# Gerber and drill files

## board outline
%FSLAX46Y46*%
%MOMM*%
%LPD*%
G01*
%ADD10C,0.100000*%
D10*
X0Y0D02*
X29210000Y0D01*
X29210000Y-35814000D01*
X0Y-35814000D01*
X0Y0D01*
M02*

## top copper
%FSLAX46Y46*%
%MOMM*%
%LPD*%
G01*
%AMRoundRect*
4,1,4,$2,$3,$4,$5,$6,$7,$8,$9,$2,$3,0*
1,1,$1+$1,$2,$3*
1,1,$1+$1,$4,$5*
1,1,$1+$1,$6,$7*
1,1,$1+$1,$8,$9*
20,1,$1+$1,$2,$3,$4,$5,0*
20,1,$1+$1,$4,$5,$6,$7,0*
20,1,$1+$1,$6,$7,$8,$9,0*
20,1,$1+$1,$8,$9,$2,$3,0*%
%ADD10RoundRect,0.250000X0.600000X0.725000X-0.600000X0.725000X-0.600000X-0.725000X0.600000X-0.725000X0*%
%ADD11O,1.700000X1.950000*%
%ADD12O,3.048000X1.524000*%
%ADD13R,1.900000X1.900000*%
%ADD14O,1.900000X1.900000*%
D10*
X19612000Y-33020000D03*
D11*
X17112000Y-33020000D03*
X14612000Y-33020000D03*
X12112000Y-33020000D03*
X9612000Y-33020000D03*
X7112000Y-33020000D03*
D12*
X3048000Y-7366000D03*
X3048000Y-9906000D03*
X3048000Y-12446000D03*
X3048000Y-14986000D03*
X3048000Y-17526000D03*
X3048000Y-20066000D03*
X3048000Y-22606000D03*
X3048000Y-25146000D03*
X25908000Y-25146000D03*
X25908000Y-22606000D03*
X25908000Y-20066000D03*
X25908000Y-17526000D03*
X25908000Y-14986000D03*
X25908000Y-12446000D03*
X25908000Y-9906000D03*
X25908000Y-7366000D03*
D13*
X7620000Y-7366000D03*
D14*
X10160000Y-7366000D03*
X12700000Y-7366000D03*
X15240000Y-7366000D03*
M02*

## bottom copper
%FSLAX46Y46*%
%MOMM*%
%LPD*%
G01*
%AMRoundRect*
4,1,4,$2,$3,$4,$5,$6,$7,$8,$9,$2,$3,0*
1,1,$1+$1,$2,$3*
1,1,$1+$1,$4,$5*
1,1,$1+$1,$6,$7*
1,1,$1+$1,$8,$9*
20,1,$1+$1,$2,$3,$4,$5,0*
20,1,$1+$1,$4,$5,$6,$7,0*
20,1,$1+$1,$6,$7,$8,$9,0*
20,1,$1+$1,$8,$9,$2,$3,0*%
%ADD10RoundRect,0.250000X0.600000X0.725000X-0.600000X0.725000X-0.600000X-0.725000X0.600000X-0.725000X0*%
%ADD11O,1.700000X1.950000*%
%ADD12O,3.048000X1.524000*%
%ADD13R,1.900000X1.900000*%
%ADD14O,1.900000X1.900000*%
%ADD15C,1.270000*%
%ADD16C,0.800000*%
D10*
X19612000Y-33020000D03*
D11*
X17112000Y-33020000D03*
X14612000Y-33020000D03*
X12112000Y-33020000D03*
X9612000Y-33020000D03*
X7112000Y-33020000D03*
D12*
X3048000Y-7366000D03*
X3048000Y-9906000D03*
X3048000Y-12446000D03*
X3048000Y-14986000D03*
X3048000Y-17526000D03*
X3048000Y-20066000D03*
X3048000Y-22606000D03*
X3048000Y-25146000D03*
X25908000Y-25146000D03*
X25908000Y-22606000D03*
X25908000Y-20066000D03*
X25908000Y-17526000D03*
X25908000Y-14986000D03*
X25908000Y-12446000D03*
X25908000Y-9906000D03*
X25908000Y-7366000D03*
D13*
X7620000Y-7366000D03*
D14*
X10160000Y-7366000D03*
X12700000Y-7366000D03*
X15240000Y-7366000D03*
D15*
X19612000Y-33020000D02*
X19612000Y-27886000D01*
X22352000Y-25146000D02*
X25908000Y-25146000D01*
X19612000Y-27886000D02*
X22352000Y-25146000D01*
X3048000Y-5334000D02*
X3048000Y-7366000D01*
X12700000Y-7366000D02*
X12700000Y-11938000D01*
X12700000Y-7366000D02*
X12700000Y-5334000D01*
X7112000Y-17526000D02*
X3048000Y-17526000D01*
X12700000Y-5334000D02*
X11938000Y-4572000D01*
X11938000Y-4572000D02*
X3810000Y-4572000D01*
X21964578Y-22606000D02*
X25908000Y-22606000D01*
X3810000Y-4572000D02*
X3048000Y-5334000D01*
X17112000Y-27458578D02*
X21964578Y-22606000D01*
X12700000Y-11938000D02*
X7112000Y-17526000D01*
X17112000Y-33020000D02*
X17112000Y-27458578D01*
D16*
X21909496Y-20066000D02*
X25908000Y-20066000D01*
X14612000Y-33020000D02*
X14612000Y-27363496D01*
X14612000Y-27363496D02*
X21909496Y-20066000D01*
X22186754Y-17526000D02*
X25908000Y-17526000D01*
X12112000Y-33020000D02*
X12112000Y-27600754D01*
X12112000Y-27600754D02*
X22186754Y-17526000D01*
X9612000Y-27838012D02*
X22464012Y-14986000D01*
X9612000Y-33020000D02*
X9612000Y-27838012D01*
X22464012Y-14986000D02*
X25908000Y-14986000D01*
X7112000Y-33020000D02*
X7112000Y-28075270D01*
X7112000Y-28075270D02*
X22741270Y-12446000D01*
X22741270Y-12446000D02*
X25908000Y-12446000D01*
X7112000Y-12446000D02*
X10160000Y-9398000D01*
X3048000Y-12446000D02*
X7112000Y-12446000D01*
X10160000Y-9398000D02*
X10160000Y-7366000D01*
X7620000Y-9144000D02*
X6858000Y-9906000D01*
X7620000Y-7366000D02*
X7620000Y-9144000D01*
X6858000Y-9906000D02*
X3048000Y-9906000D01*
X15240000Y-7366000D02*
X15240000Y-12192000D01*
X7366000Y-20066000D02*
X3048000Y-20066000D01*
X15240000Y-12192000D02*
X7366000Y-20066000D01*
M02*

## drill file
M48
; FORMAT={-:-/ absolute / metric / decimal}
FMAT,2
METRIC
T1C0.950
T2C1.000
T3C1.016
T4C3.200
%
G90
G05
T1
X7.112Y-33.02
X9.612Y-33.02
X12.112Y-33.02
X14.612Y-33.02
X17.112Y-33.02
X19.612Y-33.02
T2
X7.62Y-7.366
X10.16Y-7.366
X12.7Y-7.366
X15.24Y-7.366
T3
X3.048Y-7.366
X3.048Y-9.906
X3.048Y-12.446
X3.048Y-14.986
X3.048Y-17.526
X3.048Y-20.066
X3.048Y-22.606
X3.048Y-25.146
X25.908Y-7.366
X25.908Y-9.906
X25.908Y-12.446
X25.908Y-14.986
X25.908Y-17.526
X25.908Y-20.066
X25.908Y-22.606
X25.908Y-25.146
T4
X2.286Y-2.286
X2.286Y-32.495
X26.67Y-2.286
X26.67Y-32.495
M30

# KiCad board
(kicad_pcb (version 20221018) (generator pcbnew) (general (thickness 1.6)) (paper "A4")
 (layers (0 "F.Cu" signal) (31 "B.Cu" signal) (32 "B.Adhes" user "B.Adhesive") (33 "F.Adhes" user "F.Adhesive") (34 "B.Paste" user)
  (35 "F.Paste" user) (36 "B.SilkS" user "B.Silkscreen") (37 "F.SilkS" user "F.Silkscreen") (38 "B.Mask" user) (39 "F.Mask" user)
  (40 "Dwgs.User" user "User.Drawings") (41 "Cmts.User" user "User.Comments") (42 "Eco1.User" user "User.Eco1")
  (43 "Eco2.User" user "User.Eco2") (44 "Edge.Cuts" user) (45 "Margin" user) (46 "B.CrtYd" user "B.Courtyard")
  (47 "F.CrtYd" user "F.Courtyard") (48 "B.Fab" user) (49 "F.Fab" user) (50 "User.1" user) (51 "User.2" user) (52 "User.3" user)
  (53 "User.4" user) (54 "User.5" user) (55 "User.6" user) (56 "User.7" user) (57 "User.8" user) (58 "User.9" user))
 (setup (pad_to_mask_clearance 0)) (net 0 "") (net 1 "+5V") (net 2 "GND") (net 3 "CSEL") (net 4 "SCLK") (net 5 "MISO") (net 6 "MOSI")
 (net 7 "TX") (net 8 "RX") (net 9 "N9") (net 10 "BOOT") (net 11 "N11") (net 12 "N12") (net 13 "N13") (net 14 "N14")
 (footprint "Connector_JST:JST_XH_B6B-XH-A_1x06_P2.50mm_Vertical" (layer "F.Cu") (at 19.612 33.02 180)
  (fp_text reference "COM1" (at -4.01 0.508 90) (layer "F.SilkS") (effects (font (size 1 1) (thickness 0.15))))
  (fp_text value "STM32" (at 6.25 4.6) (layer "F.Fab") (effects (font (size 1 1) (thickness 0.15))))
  (pad "1" thru_hole roundrect (at 0 0 180) (size 1.7 1.95) (drill 0.95) (layers "*.Cu" "*.Mask") (roundrect_rratio 0.1470588235)
   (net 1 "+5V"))
  (pad "2" thru_hole oval (at 2.5 0 180) (size 1.7 1.95) (drill 0.95) (layers "*.Cu" "*.Mask") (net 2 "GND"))
  (pad "3" thru_hole oval (at 5 0 180) (size 1.7 1.95) (drill 0.95) (layers "*.Cu" "*.Mask") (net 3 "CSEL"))
  (pad "4" thru_hole oval (at 7.5 0 180) (size 1.7 1.95) (drill 0.95) (layers "*.Cu" "*.Mask") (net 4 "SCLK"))
  (pad "5" thru_hole oval (at 10 0 180) (size 1.7 1.95) (drill 0.95) (layers "*.Cu" "*.Mask") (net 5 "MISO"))
  (pad "6" thru_hole oval (at 12.5 0 180) (size 1.7 1.95) (drill 0.95) (layers "*.Cu" "*.Mask") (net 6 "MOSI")))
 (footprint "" (layer "F.Cu") (at 26.67 2.286)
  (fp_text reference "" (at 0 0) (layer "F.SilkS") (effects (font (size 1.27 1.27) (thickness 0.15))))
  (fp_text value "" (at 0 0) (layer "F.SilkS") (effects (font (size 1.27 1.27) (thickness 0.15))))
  (pad "" np_thru_hole circle (at 0 0) (size 3.2 3.2) (drill 3.2) (layers "F&B.Cu" "*.Mask")))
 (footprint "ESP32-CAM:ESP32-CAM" (layer "F.Cu") (at 14.478 14.986)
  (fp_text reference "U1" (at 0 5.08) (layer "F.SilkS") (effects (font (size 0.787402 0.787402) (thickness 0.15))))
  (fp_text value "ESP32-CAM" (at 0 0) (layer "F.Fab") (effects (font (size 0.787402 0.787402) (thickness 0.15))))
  (pad "P$1" thru_hole oval (at -11.43 -7.62) (size 3.048 1.524) (drill 1.016) (layers "*.Cu" "*.Mask") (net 2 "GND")
   (solder_mask_margin 0.102))
  (pad "P$2" thru_hole oval (at -11.43 -5.08) (size 3.048 1.524) (drill 1.016) (layers "*.Cu" "*.Mask") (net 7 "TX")
   (solder_mask_margin 0.102))
  (pad "P$3" thru_hole oval (at -11.43 -2.54) (size 3.048 1.524) (drill 1.016) (layers "*.Cu" "*.Mask") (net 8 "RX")
   (solder_mask_margin 0.102))
  (pad "P$4" thru_hole oval (at -11.43 0) (size 3.048 1.524) (drill 1.016) (layers "*.Cu" "*.Mask") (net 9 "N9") (solder_mask_margin 0.102))
  (pad "P$5" thru_hole oval (at -11.43 2.54) (size 3.048 1.524) (drill 1.016) (layers "*.Cu" "*.Mask") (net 2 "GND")
   (solder_mask_margin 0.102))
  (pad "P$6" thru_hole oval (at -11.43 5.08) (size 3.048 1.524) (drill 1.016) (layers "*.Cu" "*.Mask") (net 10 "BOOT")
   (solder_mask_margin 0.102))
  (pad "P$7" thru_hole oval (at -11.43 7.62) (size 3.048 1.524) (drill 1.016) (layers "*.Cu" "*.Mask") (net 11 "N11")
   (solder_mask_margin 0.102))
  (pad "P$8" thru_hole oval (at -11.43 10.16) (size 3.048 1.524) (drill 1.016) (layers "*.Cu" "*.Mask") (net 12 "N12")
   (solder_mask_margin 0.102))
  (pad "P$9" thru_hole oval (at 11.43 10.16) (size 3.048 1.524) (drill 1.016) (layers "*.Cu" "*.Mask") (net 1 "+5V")
   (solder_mask_margin 0.102))
  (pad "P$10" thru_hole oval (at 11.43 7.62) (size 3.048 1.524) (drill 1.016) (layers "*.Cu" "*.Mask") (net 2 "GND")
   (solder_mask_margin 0.102))
  (pad "P$11" thru_hole oval (at 11.43 5.08) (size 3.048 1.524) (drill 1.016) (layers "*.Cu" "*.Mask") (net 3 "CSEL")
   (solder_mask_margin 0.102))
  (pad "P$12" thru_hole oval (at 11.43 2.54) (size 3.048 1.524) (drill 1.016) (layers "*.Cu" "*.Mask") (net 4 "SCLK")
   (solder_mask_margin 0.102))
  (pad "P$13" thru_hole oval (at 11.43 0) (size 3.048 1.524) (drill 1.016) (layers "*.Cu" "*.Mask") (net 5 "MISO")
   (solder_mask_margin 0.102))
  (pad "P$14" thru_hole oval (at 11.43 -2.54) (size 3.048 1.524) (drill 1.016) (layers "*.Cu" "*.Mask") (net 6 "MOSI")
   (solder_mask_margin 0.102))
  (pad "P$15" thru_hole oval (at 11.43 -5.08) (size 3.048 1.524) (drill 1.016) (layers "*.Cu" "*.Mask") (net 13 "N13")
   (solder_mask_margin 0.102))
  (pad "P$16" thru_hole oval (at 11.43 -7.62) (size 3.048 1.524) (drill 1.016) (layers "*.Cu" "*.Mask") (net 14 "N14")
   (solder_mask_margin 0.102)))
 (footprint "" (layer "F.Cu") (at 2.286 2.286)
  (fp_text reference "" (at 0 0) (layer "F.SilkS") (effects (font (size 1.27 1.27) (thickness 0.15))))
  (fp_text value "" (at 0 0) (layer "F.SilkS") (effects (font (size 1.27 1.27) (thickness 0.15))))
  (pad "" np_thru_hole circle (at 0 0) (size 3.2 3.2) (drill 3.2) (layers "F&B.Cu" "*.Mask")))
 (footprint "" (layer "F.Cu") (at 26.67 32.495)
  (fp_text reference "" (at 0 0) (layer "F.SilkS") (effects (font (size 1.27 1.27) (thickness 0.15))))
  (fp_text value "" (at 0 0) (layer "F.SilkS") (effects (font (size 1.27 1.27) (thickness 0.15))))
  (pad "" np_thru_hole circle (at 0 0) (size 3.2 3.2) (drill 3.2) (layers "F&B.Cu" "*.Mask")))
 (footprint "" (layer "F.Cu") (at 2.286 32.495)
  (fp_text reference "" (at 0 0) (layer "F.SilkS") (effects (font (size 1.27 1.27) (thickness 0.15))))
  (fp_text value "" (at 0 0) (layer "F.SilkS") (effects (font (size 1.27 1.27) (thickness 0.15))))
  (pad "" np_thru_hole circle (at 0 0) (size 3.2 3.2) (drill 3.2) (layers "F&B.Cu" "*.Mask")))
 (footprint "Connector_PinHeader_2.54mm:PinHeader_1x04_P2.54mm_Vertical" (layer "F.Cu") (at 7.62 7.366 90)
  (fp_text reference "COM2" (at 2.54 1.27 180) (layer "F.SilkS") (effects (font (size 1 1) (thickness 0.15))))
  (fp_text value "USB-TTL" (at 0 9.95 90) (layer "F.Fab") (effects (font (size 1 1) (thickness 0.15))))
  (pad "1" thru_hole rect (at 0 0 90) (size 1.9 1.9) (drill 1) (layers "*.Cu" "*.Mask") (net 7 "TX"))
  (pad "2" thru_hole oval (at 0 2.54 90) (size 1.9 1.9) (drill 1) (layers "*.Cu" "*.Mask") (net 8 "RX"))
  (pad "3" thru_hole oval (at 0 5.08 90) (size 1.9 1.9) (drill 1) (layers "*.Cu" "*.Mask") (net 2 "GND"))
  (pad "4" thru_hole oval (at 0 7.62 90) (size 1.9 1.9) (drill 1) (layers "*.Cu" "*.Mask") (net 10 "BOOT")))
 (gr_rect (start 0 0) (end 29.21 35.814) (stroke (width 0.1) (type default)) (fill none) (layer "Edge.Cuts"))
 (segment (start 19.612 33.02) (end 19.612 27.886) (width 1.27) (layer "B.Cu") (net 1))
 (segment (start 22.352 25.146) (end 25.908 25.146) (width 1.27) (layer "B.Cu") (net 1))
 (segment (start 19.612 27.886) (end 22.352 25.146) (width 1.27) (layer "B.Cu") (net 1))
 (segment (start 3.048 5.334) (end 3.048 7.366) (width 1.27) (layer "B.Cu") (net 2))
 (segment (start 12.7 7.366) (end 12.7 11.938) (width 1.27) (layer "B.Cu") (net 2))
 (segment (start 12.7 7.366) (end 12.7 5.334) (width 1.27) (layer "B.Cu") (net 2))
 (segment (start 7.112 17.526) (end 3.048 17.526) (width 1.27) (layer "B.Cu") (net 2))
 (segment (start 12.7 5.334) (end 11.938 4.572) (width 1.27) (layer "B.Cu") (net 2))
 (segment (start 11.938 4.572) (end 3.81 4.572) (width 1.27) (layer "B.Cu") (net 2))
 (segment (start 21.964578 22.606) (end 25.908 22.606) (width 1.27) (layer "B.Cu") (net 2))
 (segment (start 3.81 4.572) (end 3.048 5.334) (width 1.27) (layer "B.Cu") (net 2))
 (segment (start 17.112 27.458578) (end 21.964578 22.606) (width 1.27) (layer "B.Cu") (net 2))
 (segment (start 12.7 11.938) (end 7.112 17.526) (width 1.27) (layer "B.Cu") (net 2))
 (segment (start 17.112 33.02) (end 17.112 27.458578) (width 1.27) (layer "B.Cu") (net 2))
 (segment (start 21.909496 20.066) (end 25.908 20.066) (width 0.8) (layer "B.Cu") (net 3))
 (segment (start 14.612 33.02) (end 14.612 27.363496) (width 0.8) (layer "B.Cu") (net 3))
 (segment (start 14.612 27.363496) (end 21.909496 20.066) (width 0.8) (layer "B.Cu") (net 3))
 (segment (start 22.186754 17.526) (end 25.908 17.526) (width 0.8) (layer "B.Cu") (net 4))
 (segment (start 12.112 33.02) (end 12.112 27.600754) (width 0.8) (layer "B.Cu") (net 4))
 (segment (start 12.112 27.600754) (end 22.186754 17.526) (width 0.8) (layer "B.Cu") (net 4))
 (segment (start 9.612 27.838012) (end 22.464012 14.986) (width 0.8) (layer "B.Cu") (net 5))
 (segment (start 9.612 33.02) (end 9.612 27.838012) (width 0.8) (layer "B.Cu") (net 5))
 (segment (start 22.464012 14.986) (end 25.908 14.986) (width 0.8) (layer "B.Cu") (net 5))
 (segment (start 7.112 33.02) (end 7.112 28.07527) (width 0.8) (layer "B.Cu") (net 6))
 (segment (start 7.112 28.07527) (end 22.74127 12.446) (width 0.8) (layer "B.Cu") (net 6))
 (segment (start 22.74127 12.446) (end 25.908 12.446) (width 0.8) (layer "B.Cu") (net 6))
 (segment (start 7.112 12.446) (end 10.16 9.398) (width 0.8) (layer "B.Cu") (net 8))
 (segment (start 3.048 12.446) (end 7.112 12.446) (width 0.8) (layer "B.Cu") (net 8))
 (segment (start 10.16 9.398) (end 10.16 7.366) (width 0.8) (layer "B.Cu") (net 8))
 (segment (start 7.62 9.144) (end 6.858 9.906) (width 0.8) (layer "B.Cu") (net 7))
 (segment (start 7.62 7.366) (end 7.62 9.144) (width 0.8) (layer "B.Cu") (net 7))
 (segment (start 6.858 9.906) (end 3.048 9.906) (width 0.8) (layer "B.Cu") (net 7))
 (segment (start 15.24 7.366) (end 15.24 12.192) (width 0.8) (layer "B.Cu") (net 10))
 (segment (start 7.366 20.066) (end 3.048 20.066) (width 0.8) (layer "B.Cu") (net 10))
 (segment (start 15.24 12.192) (end 7.366 20.066) (width 0.8) (layer "B.Cu") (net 10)))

